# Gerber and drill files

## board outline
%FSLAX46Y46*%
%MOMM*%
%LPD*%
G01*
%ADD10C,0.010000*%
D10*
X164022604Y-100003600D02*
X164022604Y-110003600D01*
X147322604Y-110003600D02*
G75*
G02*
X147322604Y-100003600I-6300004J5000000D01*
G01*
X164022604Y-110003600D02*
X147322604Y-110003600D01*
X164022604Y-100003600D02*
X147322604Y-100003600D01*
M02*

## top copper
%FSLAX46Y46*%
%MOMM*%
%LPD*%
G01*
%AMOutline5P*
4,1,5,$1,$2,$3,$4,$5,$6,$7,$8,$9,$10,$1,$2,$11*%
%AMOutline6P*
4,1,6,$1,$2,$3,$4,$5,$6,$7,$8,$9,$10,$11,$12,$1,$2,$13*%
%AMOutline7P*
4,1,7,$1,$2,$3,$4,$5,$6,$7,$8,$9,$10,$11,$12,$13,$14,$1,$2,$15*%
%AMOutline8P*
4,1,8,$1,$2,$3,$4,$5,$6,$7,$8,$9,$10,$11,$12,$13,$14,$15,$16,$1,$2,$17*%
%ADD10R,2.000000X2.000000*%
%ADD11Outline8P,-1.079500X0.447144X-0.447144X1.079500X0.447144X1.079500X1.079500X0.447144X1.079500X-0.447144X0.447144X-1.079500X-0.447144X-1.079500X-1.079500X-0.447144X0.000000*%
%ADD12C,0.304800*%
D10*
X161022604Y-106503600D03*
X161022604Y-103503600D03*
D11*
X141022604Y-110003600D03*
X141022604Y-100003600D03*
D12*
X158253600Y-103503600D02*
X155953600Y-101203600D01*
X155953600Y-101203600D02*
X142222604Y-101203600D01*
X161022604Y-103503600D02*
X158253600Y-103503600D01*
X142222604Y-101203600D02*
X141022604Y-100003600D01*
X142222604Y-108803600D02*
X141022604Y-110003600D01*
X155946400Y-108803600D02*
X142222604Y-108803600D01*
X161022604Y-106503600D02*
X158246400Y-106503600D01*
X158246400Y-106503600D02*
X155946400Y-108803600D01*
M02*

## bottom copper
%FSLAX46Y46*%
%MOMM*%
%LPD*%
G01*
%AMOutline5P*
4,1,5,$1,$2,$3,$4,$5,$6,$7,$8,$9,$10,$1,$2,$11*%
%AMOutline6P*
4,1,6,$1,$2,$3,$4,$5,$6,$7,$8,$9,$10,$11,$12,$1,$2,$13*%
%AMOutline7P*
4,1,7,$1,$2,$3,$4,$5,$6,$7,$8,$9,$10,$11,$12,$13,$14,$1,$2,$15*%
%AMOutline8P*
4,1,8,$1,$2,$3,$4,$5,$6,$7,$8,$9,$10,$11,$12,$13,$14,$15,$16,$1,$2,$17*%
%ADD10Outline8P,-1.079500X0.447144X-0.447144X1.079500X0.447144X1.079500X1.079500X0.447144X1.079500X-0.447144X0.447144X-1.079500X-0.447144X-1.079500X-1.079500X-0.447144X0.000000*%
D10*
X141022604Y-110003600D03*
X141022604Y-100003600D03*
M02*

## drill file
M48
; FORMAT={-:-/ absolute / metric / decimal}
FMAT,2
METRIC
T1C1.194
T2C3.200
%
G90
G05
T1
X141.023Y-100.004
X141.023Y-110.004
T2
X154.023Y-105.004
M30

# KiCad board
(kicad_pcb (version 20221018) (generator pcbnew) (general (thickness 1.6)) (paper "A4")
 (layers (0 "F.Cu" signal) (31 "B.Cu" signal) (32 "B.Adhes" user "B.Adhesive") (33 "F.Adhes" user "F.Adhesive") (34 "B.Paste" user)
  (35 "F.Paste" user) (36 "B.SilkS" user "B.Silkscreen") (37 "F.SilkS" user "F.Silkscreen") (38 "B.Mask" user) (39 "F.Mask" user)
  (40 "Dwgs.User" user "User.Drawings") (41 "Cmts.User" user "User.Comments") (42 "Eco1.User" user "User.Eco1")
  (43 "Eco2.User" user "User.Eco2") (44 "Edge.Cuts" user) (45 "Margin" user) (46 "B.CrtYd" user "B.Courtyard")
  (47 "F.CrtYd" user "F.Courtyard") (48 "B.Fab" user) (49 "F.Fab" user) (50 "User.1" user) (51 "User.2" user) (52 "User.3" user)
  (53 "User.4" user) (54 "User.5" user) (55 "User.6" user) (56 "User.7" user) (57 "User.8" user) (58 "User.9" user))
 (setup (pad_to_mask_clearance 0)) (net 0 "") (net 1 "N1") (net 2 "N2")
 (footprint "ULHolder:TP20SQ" (layer "F.Cu") (at 161.022604 106.5036)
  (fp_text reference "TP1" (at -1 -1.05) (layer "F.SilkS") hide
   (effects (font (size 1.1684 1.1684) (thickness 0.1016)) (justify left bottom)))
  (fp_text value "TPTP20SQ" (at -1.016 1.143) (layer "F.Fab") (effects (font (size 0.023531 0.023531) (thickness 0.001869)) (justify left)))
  (pad "TP" smd rect (at 0 0) (size 2 2) (layers "F.Cu" "F.Mask") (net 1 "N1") (solder_mask_margin 0.1016) (thermal_bridge_angle 45)))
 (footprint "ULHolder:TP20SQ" (layer "F.Cu") (at 161.022604 103.5036)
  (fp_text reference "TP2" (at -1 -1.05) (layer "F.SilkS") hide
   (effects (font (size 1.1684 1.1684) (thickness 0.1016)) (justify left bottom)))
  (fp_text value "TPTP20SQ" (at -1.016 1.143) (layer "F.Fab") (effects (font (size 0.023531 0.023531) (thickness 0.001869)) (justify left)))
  (pad "TP" smd rect (at 0 0) (size 2 2) (layers "F.Cu" "F.Mask") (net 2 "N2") (solder_mask_margin 0.1016) (thermal_bridge_angle 45)))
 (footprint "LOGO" (layer "F.Cu") (at 141 105 90)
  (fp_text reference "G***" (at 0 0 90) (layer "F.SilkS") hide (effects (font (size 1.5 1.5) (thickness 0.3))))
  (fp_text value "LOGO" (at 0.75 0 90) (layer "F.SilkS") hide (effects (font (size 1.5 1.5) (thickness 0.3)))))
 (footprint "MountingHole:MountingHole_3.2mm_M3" (layer "F.Cu") (at 154.022604 105.0036)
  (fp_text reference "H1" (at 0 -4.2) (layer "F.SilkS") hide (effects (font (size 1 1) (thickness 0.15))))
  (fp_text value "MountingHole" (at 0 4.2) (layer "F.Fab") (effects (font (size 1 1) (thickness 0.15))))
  (pad "" np_thru_hole circle (at 0 0) (size 3.2 3.2) (drill 3.2) (layers "*.Cu" "*.Mask")))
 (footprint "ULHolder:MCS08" (layer "F.Cu") (at 141.022604 110.0036)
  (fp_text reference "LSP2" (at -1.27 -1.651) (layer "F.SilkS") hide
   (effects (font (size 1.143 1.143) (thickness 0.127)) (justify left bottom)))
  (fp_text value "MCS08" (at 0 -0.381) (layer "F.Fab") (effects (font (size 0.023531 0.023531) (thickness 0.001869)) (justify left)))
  (pad "MP" thru_hole roundrect (at 0 0) (size 2.159 2.159) (drill 1.1938) (layers "*.Cu" "*.Mask") (roundrect_rratio 0.25)
   (chamfer_ratio 0.2928932188) (chamfer top_left top_right bottom_left bottom_right) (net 1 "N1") (solder_mask_margin 0.1016)
   (thermal_bridge_angle 45)))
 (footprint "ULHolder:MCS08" (layer "F.Cu") (at 141.022604 100.0036)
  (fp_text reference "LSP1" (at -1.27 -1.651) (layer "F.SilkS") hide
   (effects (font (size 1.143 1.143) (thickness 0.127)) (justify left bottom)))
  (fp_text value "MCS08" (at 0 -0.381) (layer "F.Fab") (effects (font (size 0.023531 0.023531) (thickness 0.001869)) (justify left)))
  (pad "MP" thru_hole roundrect (at 0 0) (size 2.159 2.159) (drill 1.1938) (layers "*.Cu" "*.Mask") (roundrect_rratio 0.25)
   (chamfer_ratio 0.2928932188) (chamfer top_left top_right bottom_left bottom_right) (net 2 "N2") (solder_mask_margin 0.1016)
   (thermal_bridge_angle 45)))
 (gr_line (start 164.022604 100.0036) (end 164.022604 110.0036) (stroke (width 0.01) (type solid)) (layer "Edge.Cuts"))
 (gr_arc (start 147.322604 110.0036) (mid 132.979595 105.0036) (end 147.322604 100.0036) (stroke (width 0.01) (type solid))
  (layer "Edge.Cuts"))
 (gr_line (start 164.022604 110.0036) (end 147.322604 110.0036) (stroke (width 0.01) (type solid)) (layer "Edge.Cuts"))
 (gr_line (start 164.022604 100.0036) (end 147.322604 100.0036) (stroke (width 0.01) (type solid)) (layer "Edge.Cuts"))
 (segment (start 158.2536 103.5036) (end 155.9536 101.2036) (width 0.3048) (layer "F.Cu") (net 2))
 (segment (start 155.9536 101.2036) (end 142.222604 101.2036) (width 0.3048) (layer "F.Cu") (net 2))
 (segment (start 161.022604 103.5036) (end 158.2536 103.5036) (width 0.3048) (layer "F.Cu") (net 2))
 (segment (start 142.222604 101.2036) (end 141.022604 100.0036) (width 0.3048) (layer "F.Cu") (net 2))
 (segment (start 142.222604 108.8036) (end 141.022604 110.0036) (width 0.3048) (layer "F.Cu") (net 1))
 (segment (start 155.9464 108.8036) (end 142.222604 108.8036) (width 0.3048) (layer "F.Cu") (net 1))
 (segment (start 161.022604 106.5036) (end 158.2464 106.5036) (width 0.3048) (layer "F.Cu") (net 1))
 (segment (start 158.2464 106.5036) (end 155.9464 108.8036) (width 0.3048) (layer "F.Cu") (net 1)))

